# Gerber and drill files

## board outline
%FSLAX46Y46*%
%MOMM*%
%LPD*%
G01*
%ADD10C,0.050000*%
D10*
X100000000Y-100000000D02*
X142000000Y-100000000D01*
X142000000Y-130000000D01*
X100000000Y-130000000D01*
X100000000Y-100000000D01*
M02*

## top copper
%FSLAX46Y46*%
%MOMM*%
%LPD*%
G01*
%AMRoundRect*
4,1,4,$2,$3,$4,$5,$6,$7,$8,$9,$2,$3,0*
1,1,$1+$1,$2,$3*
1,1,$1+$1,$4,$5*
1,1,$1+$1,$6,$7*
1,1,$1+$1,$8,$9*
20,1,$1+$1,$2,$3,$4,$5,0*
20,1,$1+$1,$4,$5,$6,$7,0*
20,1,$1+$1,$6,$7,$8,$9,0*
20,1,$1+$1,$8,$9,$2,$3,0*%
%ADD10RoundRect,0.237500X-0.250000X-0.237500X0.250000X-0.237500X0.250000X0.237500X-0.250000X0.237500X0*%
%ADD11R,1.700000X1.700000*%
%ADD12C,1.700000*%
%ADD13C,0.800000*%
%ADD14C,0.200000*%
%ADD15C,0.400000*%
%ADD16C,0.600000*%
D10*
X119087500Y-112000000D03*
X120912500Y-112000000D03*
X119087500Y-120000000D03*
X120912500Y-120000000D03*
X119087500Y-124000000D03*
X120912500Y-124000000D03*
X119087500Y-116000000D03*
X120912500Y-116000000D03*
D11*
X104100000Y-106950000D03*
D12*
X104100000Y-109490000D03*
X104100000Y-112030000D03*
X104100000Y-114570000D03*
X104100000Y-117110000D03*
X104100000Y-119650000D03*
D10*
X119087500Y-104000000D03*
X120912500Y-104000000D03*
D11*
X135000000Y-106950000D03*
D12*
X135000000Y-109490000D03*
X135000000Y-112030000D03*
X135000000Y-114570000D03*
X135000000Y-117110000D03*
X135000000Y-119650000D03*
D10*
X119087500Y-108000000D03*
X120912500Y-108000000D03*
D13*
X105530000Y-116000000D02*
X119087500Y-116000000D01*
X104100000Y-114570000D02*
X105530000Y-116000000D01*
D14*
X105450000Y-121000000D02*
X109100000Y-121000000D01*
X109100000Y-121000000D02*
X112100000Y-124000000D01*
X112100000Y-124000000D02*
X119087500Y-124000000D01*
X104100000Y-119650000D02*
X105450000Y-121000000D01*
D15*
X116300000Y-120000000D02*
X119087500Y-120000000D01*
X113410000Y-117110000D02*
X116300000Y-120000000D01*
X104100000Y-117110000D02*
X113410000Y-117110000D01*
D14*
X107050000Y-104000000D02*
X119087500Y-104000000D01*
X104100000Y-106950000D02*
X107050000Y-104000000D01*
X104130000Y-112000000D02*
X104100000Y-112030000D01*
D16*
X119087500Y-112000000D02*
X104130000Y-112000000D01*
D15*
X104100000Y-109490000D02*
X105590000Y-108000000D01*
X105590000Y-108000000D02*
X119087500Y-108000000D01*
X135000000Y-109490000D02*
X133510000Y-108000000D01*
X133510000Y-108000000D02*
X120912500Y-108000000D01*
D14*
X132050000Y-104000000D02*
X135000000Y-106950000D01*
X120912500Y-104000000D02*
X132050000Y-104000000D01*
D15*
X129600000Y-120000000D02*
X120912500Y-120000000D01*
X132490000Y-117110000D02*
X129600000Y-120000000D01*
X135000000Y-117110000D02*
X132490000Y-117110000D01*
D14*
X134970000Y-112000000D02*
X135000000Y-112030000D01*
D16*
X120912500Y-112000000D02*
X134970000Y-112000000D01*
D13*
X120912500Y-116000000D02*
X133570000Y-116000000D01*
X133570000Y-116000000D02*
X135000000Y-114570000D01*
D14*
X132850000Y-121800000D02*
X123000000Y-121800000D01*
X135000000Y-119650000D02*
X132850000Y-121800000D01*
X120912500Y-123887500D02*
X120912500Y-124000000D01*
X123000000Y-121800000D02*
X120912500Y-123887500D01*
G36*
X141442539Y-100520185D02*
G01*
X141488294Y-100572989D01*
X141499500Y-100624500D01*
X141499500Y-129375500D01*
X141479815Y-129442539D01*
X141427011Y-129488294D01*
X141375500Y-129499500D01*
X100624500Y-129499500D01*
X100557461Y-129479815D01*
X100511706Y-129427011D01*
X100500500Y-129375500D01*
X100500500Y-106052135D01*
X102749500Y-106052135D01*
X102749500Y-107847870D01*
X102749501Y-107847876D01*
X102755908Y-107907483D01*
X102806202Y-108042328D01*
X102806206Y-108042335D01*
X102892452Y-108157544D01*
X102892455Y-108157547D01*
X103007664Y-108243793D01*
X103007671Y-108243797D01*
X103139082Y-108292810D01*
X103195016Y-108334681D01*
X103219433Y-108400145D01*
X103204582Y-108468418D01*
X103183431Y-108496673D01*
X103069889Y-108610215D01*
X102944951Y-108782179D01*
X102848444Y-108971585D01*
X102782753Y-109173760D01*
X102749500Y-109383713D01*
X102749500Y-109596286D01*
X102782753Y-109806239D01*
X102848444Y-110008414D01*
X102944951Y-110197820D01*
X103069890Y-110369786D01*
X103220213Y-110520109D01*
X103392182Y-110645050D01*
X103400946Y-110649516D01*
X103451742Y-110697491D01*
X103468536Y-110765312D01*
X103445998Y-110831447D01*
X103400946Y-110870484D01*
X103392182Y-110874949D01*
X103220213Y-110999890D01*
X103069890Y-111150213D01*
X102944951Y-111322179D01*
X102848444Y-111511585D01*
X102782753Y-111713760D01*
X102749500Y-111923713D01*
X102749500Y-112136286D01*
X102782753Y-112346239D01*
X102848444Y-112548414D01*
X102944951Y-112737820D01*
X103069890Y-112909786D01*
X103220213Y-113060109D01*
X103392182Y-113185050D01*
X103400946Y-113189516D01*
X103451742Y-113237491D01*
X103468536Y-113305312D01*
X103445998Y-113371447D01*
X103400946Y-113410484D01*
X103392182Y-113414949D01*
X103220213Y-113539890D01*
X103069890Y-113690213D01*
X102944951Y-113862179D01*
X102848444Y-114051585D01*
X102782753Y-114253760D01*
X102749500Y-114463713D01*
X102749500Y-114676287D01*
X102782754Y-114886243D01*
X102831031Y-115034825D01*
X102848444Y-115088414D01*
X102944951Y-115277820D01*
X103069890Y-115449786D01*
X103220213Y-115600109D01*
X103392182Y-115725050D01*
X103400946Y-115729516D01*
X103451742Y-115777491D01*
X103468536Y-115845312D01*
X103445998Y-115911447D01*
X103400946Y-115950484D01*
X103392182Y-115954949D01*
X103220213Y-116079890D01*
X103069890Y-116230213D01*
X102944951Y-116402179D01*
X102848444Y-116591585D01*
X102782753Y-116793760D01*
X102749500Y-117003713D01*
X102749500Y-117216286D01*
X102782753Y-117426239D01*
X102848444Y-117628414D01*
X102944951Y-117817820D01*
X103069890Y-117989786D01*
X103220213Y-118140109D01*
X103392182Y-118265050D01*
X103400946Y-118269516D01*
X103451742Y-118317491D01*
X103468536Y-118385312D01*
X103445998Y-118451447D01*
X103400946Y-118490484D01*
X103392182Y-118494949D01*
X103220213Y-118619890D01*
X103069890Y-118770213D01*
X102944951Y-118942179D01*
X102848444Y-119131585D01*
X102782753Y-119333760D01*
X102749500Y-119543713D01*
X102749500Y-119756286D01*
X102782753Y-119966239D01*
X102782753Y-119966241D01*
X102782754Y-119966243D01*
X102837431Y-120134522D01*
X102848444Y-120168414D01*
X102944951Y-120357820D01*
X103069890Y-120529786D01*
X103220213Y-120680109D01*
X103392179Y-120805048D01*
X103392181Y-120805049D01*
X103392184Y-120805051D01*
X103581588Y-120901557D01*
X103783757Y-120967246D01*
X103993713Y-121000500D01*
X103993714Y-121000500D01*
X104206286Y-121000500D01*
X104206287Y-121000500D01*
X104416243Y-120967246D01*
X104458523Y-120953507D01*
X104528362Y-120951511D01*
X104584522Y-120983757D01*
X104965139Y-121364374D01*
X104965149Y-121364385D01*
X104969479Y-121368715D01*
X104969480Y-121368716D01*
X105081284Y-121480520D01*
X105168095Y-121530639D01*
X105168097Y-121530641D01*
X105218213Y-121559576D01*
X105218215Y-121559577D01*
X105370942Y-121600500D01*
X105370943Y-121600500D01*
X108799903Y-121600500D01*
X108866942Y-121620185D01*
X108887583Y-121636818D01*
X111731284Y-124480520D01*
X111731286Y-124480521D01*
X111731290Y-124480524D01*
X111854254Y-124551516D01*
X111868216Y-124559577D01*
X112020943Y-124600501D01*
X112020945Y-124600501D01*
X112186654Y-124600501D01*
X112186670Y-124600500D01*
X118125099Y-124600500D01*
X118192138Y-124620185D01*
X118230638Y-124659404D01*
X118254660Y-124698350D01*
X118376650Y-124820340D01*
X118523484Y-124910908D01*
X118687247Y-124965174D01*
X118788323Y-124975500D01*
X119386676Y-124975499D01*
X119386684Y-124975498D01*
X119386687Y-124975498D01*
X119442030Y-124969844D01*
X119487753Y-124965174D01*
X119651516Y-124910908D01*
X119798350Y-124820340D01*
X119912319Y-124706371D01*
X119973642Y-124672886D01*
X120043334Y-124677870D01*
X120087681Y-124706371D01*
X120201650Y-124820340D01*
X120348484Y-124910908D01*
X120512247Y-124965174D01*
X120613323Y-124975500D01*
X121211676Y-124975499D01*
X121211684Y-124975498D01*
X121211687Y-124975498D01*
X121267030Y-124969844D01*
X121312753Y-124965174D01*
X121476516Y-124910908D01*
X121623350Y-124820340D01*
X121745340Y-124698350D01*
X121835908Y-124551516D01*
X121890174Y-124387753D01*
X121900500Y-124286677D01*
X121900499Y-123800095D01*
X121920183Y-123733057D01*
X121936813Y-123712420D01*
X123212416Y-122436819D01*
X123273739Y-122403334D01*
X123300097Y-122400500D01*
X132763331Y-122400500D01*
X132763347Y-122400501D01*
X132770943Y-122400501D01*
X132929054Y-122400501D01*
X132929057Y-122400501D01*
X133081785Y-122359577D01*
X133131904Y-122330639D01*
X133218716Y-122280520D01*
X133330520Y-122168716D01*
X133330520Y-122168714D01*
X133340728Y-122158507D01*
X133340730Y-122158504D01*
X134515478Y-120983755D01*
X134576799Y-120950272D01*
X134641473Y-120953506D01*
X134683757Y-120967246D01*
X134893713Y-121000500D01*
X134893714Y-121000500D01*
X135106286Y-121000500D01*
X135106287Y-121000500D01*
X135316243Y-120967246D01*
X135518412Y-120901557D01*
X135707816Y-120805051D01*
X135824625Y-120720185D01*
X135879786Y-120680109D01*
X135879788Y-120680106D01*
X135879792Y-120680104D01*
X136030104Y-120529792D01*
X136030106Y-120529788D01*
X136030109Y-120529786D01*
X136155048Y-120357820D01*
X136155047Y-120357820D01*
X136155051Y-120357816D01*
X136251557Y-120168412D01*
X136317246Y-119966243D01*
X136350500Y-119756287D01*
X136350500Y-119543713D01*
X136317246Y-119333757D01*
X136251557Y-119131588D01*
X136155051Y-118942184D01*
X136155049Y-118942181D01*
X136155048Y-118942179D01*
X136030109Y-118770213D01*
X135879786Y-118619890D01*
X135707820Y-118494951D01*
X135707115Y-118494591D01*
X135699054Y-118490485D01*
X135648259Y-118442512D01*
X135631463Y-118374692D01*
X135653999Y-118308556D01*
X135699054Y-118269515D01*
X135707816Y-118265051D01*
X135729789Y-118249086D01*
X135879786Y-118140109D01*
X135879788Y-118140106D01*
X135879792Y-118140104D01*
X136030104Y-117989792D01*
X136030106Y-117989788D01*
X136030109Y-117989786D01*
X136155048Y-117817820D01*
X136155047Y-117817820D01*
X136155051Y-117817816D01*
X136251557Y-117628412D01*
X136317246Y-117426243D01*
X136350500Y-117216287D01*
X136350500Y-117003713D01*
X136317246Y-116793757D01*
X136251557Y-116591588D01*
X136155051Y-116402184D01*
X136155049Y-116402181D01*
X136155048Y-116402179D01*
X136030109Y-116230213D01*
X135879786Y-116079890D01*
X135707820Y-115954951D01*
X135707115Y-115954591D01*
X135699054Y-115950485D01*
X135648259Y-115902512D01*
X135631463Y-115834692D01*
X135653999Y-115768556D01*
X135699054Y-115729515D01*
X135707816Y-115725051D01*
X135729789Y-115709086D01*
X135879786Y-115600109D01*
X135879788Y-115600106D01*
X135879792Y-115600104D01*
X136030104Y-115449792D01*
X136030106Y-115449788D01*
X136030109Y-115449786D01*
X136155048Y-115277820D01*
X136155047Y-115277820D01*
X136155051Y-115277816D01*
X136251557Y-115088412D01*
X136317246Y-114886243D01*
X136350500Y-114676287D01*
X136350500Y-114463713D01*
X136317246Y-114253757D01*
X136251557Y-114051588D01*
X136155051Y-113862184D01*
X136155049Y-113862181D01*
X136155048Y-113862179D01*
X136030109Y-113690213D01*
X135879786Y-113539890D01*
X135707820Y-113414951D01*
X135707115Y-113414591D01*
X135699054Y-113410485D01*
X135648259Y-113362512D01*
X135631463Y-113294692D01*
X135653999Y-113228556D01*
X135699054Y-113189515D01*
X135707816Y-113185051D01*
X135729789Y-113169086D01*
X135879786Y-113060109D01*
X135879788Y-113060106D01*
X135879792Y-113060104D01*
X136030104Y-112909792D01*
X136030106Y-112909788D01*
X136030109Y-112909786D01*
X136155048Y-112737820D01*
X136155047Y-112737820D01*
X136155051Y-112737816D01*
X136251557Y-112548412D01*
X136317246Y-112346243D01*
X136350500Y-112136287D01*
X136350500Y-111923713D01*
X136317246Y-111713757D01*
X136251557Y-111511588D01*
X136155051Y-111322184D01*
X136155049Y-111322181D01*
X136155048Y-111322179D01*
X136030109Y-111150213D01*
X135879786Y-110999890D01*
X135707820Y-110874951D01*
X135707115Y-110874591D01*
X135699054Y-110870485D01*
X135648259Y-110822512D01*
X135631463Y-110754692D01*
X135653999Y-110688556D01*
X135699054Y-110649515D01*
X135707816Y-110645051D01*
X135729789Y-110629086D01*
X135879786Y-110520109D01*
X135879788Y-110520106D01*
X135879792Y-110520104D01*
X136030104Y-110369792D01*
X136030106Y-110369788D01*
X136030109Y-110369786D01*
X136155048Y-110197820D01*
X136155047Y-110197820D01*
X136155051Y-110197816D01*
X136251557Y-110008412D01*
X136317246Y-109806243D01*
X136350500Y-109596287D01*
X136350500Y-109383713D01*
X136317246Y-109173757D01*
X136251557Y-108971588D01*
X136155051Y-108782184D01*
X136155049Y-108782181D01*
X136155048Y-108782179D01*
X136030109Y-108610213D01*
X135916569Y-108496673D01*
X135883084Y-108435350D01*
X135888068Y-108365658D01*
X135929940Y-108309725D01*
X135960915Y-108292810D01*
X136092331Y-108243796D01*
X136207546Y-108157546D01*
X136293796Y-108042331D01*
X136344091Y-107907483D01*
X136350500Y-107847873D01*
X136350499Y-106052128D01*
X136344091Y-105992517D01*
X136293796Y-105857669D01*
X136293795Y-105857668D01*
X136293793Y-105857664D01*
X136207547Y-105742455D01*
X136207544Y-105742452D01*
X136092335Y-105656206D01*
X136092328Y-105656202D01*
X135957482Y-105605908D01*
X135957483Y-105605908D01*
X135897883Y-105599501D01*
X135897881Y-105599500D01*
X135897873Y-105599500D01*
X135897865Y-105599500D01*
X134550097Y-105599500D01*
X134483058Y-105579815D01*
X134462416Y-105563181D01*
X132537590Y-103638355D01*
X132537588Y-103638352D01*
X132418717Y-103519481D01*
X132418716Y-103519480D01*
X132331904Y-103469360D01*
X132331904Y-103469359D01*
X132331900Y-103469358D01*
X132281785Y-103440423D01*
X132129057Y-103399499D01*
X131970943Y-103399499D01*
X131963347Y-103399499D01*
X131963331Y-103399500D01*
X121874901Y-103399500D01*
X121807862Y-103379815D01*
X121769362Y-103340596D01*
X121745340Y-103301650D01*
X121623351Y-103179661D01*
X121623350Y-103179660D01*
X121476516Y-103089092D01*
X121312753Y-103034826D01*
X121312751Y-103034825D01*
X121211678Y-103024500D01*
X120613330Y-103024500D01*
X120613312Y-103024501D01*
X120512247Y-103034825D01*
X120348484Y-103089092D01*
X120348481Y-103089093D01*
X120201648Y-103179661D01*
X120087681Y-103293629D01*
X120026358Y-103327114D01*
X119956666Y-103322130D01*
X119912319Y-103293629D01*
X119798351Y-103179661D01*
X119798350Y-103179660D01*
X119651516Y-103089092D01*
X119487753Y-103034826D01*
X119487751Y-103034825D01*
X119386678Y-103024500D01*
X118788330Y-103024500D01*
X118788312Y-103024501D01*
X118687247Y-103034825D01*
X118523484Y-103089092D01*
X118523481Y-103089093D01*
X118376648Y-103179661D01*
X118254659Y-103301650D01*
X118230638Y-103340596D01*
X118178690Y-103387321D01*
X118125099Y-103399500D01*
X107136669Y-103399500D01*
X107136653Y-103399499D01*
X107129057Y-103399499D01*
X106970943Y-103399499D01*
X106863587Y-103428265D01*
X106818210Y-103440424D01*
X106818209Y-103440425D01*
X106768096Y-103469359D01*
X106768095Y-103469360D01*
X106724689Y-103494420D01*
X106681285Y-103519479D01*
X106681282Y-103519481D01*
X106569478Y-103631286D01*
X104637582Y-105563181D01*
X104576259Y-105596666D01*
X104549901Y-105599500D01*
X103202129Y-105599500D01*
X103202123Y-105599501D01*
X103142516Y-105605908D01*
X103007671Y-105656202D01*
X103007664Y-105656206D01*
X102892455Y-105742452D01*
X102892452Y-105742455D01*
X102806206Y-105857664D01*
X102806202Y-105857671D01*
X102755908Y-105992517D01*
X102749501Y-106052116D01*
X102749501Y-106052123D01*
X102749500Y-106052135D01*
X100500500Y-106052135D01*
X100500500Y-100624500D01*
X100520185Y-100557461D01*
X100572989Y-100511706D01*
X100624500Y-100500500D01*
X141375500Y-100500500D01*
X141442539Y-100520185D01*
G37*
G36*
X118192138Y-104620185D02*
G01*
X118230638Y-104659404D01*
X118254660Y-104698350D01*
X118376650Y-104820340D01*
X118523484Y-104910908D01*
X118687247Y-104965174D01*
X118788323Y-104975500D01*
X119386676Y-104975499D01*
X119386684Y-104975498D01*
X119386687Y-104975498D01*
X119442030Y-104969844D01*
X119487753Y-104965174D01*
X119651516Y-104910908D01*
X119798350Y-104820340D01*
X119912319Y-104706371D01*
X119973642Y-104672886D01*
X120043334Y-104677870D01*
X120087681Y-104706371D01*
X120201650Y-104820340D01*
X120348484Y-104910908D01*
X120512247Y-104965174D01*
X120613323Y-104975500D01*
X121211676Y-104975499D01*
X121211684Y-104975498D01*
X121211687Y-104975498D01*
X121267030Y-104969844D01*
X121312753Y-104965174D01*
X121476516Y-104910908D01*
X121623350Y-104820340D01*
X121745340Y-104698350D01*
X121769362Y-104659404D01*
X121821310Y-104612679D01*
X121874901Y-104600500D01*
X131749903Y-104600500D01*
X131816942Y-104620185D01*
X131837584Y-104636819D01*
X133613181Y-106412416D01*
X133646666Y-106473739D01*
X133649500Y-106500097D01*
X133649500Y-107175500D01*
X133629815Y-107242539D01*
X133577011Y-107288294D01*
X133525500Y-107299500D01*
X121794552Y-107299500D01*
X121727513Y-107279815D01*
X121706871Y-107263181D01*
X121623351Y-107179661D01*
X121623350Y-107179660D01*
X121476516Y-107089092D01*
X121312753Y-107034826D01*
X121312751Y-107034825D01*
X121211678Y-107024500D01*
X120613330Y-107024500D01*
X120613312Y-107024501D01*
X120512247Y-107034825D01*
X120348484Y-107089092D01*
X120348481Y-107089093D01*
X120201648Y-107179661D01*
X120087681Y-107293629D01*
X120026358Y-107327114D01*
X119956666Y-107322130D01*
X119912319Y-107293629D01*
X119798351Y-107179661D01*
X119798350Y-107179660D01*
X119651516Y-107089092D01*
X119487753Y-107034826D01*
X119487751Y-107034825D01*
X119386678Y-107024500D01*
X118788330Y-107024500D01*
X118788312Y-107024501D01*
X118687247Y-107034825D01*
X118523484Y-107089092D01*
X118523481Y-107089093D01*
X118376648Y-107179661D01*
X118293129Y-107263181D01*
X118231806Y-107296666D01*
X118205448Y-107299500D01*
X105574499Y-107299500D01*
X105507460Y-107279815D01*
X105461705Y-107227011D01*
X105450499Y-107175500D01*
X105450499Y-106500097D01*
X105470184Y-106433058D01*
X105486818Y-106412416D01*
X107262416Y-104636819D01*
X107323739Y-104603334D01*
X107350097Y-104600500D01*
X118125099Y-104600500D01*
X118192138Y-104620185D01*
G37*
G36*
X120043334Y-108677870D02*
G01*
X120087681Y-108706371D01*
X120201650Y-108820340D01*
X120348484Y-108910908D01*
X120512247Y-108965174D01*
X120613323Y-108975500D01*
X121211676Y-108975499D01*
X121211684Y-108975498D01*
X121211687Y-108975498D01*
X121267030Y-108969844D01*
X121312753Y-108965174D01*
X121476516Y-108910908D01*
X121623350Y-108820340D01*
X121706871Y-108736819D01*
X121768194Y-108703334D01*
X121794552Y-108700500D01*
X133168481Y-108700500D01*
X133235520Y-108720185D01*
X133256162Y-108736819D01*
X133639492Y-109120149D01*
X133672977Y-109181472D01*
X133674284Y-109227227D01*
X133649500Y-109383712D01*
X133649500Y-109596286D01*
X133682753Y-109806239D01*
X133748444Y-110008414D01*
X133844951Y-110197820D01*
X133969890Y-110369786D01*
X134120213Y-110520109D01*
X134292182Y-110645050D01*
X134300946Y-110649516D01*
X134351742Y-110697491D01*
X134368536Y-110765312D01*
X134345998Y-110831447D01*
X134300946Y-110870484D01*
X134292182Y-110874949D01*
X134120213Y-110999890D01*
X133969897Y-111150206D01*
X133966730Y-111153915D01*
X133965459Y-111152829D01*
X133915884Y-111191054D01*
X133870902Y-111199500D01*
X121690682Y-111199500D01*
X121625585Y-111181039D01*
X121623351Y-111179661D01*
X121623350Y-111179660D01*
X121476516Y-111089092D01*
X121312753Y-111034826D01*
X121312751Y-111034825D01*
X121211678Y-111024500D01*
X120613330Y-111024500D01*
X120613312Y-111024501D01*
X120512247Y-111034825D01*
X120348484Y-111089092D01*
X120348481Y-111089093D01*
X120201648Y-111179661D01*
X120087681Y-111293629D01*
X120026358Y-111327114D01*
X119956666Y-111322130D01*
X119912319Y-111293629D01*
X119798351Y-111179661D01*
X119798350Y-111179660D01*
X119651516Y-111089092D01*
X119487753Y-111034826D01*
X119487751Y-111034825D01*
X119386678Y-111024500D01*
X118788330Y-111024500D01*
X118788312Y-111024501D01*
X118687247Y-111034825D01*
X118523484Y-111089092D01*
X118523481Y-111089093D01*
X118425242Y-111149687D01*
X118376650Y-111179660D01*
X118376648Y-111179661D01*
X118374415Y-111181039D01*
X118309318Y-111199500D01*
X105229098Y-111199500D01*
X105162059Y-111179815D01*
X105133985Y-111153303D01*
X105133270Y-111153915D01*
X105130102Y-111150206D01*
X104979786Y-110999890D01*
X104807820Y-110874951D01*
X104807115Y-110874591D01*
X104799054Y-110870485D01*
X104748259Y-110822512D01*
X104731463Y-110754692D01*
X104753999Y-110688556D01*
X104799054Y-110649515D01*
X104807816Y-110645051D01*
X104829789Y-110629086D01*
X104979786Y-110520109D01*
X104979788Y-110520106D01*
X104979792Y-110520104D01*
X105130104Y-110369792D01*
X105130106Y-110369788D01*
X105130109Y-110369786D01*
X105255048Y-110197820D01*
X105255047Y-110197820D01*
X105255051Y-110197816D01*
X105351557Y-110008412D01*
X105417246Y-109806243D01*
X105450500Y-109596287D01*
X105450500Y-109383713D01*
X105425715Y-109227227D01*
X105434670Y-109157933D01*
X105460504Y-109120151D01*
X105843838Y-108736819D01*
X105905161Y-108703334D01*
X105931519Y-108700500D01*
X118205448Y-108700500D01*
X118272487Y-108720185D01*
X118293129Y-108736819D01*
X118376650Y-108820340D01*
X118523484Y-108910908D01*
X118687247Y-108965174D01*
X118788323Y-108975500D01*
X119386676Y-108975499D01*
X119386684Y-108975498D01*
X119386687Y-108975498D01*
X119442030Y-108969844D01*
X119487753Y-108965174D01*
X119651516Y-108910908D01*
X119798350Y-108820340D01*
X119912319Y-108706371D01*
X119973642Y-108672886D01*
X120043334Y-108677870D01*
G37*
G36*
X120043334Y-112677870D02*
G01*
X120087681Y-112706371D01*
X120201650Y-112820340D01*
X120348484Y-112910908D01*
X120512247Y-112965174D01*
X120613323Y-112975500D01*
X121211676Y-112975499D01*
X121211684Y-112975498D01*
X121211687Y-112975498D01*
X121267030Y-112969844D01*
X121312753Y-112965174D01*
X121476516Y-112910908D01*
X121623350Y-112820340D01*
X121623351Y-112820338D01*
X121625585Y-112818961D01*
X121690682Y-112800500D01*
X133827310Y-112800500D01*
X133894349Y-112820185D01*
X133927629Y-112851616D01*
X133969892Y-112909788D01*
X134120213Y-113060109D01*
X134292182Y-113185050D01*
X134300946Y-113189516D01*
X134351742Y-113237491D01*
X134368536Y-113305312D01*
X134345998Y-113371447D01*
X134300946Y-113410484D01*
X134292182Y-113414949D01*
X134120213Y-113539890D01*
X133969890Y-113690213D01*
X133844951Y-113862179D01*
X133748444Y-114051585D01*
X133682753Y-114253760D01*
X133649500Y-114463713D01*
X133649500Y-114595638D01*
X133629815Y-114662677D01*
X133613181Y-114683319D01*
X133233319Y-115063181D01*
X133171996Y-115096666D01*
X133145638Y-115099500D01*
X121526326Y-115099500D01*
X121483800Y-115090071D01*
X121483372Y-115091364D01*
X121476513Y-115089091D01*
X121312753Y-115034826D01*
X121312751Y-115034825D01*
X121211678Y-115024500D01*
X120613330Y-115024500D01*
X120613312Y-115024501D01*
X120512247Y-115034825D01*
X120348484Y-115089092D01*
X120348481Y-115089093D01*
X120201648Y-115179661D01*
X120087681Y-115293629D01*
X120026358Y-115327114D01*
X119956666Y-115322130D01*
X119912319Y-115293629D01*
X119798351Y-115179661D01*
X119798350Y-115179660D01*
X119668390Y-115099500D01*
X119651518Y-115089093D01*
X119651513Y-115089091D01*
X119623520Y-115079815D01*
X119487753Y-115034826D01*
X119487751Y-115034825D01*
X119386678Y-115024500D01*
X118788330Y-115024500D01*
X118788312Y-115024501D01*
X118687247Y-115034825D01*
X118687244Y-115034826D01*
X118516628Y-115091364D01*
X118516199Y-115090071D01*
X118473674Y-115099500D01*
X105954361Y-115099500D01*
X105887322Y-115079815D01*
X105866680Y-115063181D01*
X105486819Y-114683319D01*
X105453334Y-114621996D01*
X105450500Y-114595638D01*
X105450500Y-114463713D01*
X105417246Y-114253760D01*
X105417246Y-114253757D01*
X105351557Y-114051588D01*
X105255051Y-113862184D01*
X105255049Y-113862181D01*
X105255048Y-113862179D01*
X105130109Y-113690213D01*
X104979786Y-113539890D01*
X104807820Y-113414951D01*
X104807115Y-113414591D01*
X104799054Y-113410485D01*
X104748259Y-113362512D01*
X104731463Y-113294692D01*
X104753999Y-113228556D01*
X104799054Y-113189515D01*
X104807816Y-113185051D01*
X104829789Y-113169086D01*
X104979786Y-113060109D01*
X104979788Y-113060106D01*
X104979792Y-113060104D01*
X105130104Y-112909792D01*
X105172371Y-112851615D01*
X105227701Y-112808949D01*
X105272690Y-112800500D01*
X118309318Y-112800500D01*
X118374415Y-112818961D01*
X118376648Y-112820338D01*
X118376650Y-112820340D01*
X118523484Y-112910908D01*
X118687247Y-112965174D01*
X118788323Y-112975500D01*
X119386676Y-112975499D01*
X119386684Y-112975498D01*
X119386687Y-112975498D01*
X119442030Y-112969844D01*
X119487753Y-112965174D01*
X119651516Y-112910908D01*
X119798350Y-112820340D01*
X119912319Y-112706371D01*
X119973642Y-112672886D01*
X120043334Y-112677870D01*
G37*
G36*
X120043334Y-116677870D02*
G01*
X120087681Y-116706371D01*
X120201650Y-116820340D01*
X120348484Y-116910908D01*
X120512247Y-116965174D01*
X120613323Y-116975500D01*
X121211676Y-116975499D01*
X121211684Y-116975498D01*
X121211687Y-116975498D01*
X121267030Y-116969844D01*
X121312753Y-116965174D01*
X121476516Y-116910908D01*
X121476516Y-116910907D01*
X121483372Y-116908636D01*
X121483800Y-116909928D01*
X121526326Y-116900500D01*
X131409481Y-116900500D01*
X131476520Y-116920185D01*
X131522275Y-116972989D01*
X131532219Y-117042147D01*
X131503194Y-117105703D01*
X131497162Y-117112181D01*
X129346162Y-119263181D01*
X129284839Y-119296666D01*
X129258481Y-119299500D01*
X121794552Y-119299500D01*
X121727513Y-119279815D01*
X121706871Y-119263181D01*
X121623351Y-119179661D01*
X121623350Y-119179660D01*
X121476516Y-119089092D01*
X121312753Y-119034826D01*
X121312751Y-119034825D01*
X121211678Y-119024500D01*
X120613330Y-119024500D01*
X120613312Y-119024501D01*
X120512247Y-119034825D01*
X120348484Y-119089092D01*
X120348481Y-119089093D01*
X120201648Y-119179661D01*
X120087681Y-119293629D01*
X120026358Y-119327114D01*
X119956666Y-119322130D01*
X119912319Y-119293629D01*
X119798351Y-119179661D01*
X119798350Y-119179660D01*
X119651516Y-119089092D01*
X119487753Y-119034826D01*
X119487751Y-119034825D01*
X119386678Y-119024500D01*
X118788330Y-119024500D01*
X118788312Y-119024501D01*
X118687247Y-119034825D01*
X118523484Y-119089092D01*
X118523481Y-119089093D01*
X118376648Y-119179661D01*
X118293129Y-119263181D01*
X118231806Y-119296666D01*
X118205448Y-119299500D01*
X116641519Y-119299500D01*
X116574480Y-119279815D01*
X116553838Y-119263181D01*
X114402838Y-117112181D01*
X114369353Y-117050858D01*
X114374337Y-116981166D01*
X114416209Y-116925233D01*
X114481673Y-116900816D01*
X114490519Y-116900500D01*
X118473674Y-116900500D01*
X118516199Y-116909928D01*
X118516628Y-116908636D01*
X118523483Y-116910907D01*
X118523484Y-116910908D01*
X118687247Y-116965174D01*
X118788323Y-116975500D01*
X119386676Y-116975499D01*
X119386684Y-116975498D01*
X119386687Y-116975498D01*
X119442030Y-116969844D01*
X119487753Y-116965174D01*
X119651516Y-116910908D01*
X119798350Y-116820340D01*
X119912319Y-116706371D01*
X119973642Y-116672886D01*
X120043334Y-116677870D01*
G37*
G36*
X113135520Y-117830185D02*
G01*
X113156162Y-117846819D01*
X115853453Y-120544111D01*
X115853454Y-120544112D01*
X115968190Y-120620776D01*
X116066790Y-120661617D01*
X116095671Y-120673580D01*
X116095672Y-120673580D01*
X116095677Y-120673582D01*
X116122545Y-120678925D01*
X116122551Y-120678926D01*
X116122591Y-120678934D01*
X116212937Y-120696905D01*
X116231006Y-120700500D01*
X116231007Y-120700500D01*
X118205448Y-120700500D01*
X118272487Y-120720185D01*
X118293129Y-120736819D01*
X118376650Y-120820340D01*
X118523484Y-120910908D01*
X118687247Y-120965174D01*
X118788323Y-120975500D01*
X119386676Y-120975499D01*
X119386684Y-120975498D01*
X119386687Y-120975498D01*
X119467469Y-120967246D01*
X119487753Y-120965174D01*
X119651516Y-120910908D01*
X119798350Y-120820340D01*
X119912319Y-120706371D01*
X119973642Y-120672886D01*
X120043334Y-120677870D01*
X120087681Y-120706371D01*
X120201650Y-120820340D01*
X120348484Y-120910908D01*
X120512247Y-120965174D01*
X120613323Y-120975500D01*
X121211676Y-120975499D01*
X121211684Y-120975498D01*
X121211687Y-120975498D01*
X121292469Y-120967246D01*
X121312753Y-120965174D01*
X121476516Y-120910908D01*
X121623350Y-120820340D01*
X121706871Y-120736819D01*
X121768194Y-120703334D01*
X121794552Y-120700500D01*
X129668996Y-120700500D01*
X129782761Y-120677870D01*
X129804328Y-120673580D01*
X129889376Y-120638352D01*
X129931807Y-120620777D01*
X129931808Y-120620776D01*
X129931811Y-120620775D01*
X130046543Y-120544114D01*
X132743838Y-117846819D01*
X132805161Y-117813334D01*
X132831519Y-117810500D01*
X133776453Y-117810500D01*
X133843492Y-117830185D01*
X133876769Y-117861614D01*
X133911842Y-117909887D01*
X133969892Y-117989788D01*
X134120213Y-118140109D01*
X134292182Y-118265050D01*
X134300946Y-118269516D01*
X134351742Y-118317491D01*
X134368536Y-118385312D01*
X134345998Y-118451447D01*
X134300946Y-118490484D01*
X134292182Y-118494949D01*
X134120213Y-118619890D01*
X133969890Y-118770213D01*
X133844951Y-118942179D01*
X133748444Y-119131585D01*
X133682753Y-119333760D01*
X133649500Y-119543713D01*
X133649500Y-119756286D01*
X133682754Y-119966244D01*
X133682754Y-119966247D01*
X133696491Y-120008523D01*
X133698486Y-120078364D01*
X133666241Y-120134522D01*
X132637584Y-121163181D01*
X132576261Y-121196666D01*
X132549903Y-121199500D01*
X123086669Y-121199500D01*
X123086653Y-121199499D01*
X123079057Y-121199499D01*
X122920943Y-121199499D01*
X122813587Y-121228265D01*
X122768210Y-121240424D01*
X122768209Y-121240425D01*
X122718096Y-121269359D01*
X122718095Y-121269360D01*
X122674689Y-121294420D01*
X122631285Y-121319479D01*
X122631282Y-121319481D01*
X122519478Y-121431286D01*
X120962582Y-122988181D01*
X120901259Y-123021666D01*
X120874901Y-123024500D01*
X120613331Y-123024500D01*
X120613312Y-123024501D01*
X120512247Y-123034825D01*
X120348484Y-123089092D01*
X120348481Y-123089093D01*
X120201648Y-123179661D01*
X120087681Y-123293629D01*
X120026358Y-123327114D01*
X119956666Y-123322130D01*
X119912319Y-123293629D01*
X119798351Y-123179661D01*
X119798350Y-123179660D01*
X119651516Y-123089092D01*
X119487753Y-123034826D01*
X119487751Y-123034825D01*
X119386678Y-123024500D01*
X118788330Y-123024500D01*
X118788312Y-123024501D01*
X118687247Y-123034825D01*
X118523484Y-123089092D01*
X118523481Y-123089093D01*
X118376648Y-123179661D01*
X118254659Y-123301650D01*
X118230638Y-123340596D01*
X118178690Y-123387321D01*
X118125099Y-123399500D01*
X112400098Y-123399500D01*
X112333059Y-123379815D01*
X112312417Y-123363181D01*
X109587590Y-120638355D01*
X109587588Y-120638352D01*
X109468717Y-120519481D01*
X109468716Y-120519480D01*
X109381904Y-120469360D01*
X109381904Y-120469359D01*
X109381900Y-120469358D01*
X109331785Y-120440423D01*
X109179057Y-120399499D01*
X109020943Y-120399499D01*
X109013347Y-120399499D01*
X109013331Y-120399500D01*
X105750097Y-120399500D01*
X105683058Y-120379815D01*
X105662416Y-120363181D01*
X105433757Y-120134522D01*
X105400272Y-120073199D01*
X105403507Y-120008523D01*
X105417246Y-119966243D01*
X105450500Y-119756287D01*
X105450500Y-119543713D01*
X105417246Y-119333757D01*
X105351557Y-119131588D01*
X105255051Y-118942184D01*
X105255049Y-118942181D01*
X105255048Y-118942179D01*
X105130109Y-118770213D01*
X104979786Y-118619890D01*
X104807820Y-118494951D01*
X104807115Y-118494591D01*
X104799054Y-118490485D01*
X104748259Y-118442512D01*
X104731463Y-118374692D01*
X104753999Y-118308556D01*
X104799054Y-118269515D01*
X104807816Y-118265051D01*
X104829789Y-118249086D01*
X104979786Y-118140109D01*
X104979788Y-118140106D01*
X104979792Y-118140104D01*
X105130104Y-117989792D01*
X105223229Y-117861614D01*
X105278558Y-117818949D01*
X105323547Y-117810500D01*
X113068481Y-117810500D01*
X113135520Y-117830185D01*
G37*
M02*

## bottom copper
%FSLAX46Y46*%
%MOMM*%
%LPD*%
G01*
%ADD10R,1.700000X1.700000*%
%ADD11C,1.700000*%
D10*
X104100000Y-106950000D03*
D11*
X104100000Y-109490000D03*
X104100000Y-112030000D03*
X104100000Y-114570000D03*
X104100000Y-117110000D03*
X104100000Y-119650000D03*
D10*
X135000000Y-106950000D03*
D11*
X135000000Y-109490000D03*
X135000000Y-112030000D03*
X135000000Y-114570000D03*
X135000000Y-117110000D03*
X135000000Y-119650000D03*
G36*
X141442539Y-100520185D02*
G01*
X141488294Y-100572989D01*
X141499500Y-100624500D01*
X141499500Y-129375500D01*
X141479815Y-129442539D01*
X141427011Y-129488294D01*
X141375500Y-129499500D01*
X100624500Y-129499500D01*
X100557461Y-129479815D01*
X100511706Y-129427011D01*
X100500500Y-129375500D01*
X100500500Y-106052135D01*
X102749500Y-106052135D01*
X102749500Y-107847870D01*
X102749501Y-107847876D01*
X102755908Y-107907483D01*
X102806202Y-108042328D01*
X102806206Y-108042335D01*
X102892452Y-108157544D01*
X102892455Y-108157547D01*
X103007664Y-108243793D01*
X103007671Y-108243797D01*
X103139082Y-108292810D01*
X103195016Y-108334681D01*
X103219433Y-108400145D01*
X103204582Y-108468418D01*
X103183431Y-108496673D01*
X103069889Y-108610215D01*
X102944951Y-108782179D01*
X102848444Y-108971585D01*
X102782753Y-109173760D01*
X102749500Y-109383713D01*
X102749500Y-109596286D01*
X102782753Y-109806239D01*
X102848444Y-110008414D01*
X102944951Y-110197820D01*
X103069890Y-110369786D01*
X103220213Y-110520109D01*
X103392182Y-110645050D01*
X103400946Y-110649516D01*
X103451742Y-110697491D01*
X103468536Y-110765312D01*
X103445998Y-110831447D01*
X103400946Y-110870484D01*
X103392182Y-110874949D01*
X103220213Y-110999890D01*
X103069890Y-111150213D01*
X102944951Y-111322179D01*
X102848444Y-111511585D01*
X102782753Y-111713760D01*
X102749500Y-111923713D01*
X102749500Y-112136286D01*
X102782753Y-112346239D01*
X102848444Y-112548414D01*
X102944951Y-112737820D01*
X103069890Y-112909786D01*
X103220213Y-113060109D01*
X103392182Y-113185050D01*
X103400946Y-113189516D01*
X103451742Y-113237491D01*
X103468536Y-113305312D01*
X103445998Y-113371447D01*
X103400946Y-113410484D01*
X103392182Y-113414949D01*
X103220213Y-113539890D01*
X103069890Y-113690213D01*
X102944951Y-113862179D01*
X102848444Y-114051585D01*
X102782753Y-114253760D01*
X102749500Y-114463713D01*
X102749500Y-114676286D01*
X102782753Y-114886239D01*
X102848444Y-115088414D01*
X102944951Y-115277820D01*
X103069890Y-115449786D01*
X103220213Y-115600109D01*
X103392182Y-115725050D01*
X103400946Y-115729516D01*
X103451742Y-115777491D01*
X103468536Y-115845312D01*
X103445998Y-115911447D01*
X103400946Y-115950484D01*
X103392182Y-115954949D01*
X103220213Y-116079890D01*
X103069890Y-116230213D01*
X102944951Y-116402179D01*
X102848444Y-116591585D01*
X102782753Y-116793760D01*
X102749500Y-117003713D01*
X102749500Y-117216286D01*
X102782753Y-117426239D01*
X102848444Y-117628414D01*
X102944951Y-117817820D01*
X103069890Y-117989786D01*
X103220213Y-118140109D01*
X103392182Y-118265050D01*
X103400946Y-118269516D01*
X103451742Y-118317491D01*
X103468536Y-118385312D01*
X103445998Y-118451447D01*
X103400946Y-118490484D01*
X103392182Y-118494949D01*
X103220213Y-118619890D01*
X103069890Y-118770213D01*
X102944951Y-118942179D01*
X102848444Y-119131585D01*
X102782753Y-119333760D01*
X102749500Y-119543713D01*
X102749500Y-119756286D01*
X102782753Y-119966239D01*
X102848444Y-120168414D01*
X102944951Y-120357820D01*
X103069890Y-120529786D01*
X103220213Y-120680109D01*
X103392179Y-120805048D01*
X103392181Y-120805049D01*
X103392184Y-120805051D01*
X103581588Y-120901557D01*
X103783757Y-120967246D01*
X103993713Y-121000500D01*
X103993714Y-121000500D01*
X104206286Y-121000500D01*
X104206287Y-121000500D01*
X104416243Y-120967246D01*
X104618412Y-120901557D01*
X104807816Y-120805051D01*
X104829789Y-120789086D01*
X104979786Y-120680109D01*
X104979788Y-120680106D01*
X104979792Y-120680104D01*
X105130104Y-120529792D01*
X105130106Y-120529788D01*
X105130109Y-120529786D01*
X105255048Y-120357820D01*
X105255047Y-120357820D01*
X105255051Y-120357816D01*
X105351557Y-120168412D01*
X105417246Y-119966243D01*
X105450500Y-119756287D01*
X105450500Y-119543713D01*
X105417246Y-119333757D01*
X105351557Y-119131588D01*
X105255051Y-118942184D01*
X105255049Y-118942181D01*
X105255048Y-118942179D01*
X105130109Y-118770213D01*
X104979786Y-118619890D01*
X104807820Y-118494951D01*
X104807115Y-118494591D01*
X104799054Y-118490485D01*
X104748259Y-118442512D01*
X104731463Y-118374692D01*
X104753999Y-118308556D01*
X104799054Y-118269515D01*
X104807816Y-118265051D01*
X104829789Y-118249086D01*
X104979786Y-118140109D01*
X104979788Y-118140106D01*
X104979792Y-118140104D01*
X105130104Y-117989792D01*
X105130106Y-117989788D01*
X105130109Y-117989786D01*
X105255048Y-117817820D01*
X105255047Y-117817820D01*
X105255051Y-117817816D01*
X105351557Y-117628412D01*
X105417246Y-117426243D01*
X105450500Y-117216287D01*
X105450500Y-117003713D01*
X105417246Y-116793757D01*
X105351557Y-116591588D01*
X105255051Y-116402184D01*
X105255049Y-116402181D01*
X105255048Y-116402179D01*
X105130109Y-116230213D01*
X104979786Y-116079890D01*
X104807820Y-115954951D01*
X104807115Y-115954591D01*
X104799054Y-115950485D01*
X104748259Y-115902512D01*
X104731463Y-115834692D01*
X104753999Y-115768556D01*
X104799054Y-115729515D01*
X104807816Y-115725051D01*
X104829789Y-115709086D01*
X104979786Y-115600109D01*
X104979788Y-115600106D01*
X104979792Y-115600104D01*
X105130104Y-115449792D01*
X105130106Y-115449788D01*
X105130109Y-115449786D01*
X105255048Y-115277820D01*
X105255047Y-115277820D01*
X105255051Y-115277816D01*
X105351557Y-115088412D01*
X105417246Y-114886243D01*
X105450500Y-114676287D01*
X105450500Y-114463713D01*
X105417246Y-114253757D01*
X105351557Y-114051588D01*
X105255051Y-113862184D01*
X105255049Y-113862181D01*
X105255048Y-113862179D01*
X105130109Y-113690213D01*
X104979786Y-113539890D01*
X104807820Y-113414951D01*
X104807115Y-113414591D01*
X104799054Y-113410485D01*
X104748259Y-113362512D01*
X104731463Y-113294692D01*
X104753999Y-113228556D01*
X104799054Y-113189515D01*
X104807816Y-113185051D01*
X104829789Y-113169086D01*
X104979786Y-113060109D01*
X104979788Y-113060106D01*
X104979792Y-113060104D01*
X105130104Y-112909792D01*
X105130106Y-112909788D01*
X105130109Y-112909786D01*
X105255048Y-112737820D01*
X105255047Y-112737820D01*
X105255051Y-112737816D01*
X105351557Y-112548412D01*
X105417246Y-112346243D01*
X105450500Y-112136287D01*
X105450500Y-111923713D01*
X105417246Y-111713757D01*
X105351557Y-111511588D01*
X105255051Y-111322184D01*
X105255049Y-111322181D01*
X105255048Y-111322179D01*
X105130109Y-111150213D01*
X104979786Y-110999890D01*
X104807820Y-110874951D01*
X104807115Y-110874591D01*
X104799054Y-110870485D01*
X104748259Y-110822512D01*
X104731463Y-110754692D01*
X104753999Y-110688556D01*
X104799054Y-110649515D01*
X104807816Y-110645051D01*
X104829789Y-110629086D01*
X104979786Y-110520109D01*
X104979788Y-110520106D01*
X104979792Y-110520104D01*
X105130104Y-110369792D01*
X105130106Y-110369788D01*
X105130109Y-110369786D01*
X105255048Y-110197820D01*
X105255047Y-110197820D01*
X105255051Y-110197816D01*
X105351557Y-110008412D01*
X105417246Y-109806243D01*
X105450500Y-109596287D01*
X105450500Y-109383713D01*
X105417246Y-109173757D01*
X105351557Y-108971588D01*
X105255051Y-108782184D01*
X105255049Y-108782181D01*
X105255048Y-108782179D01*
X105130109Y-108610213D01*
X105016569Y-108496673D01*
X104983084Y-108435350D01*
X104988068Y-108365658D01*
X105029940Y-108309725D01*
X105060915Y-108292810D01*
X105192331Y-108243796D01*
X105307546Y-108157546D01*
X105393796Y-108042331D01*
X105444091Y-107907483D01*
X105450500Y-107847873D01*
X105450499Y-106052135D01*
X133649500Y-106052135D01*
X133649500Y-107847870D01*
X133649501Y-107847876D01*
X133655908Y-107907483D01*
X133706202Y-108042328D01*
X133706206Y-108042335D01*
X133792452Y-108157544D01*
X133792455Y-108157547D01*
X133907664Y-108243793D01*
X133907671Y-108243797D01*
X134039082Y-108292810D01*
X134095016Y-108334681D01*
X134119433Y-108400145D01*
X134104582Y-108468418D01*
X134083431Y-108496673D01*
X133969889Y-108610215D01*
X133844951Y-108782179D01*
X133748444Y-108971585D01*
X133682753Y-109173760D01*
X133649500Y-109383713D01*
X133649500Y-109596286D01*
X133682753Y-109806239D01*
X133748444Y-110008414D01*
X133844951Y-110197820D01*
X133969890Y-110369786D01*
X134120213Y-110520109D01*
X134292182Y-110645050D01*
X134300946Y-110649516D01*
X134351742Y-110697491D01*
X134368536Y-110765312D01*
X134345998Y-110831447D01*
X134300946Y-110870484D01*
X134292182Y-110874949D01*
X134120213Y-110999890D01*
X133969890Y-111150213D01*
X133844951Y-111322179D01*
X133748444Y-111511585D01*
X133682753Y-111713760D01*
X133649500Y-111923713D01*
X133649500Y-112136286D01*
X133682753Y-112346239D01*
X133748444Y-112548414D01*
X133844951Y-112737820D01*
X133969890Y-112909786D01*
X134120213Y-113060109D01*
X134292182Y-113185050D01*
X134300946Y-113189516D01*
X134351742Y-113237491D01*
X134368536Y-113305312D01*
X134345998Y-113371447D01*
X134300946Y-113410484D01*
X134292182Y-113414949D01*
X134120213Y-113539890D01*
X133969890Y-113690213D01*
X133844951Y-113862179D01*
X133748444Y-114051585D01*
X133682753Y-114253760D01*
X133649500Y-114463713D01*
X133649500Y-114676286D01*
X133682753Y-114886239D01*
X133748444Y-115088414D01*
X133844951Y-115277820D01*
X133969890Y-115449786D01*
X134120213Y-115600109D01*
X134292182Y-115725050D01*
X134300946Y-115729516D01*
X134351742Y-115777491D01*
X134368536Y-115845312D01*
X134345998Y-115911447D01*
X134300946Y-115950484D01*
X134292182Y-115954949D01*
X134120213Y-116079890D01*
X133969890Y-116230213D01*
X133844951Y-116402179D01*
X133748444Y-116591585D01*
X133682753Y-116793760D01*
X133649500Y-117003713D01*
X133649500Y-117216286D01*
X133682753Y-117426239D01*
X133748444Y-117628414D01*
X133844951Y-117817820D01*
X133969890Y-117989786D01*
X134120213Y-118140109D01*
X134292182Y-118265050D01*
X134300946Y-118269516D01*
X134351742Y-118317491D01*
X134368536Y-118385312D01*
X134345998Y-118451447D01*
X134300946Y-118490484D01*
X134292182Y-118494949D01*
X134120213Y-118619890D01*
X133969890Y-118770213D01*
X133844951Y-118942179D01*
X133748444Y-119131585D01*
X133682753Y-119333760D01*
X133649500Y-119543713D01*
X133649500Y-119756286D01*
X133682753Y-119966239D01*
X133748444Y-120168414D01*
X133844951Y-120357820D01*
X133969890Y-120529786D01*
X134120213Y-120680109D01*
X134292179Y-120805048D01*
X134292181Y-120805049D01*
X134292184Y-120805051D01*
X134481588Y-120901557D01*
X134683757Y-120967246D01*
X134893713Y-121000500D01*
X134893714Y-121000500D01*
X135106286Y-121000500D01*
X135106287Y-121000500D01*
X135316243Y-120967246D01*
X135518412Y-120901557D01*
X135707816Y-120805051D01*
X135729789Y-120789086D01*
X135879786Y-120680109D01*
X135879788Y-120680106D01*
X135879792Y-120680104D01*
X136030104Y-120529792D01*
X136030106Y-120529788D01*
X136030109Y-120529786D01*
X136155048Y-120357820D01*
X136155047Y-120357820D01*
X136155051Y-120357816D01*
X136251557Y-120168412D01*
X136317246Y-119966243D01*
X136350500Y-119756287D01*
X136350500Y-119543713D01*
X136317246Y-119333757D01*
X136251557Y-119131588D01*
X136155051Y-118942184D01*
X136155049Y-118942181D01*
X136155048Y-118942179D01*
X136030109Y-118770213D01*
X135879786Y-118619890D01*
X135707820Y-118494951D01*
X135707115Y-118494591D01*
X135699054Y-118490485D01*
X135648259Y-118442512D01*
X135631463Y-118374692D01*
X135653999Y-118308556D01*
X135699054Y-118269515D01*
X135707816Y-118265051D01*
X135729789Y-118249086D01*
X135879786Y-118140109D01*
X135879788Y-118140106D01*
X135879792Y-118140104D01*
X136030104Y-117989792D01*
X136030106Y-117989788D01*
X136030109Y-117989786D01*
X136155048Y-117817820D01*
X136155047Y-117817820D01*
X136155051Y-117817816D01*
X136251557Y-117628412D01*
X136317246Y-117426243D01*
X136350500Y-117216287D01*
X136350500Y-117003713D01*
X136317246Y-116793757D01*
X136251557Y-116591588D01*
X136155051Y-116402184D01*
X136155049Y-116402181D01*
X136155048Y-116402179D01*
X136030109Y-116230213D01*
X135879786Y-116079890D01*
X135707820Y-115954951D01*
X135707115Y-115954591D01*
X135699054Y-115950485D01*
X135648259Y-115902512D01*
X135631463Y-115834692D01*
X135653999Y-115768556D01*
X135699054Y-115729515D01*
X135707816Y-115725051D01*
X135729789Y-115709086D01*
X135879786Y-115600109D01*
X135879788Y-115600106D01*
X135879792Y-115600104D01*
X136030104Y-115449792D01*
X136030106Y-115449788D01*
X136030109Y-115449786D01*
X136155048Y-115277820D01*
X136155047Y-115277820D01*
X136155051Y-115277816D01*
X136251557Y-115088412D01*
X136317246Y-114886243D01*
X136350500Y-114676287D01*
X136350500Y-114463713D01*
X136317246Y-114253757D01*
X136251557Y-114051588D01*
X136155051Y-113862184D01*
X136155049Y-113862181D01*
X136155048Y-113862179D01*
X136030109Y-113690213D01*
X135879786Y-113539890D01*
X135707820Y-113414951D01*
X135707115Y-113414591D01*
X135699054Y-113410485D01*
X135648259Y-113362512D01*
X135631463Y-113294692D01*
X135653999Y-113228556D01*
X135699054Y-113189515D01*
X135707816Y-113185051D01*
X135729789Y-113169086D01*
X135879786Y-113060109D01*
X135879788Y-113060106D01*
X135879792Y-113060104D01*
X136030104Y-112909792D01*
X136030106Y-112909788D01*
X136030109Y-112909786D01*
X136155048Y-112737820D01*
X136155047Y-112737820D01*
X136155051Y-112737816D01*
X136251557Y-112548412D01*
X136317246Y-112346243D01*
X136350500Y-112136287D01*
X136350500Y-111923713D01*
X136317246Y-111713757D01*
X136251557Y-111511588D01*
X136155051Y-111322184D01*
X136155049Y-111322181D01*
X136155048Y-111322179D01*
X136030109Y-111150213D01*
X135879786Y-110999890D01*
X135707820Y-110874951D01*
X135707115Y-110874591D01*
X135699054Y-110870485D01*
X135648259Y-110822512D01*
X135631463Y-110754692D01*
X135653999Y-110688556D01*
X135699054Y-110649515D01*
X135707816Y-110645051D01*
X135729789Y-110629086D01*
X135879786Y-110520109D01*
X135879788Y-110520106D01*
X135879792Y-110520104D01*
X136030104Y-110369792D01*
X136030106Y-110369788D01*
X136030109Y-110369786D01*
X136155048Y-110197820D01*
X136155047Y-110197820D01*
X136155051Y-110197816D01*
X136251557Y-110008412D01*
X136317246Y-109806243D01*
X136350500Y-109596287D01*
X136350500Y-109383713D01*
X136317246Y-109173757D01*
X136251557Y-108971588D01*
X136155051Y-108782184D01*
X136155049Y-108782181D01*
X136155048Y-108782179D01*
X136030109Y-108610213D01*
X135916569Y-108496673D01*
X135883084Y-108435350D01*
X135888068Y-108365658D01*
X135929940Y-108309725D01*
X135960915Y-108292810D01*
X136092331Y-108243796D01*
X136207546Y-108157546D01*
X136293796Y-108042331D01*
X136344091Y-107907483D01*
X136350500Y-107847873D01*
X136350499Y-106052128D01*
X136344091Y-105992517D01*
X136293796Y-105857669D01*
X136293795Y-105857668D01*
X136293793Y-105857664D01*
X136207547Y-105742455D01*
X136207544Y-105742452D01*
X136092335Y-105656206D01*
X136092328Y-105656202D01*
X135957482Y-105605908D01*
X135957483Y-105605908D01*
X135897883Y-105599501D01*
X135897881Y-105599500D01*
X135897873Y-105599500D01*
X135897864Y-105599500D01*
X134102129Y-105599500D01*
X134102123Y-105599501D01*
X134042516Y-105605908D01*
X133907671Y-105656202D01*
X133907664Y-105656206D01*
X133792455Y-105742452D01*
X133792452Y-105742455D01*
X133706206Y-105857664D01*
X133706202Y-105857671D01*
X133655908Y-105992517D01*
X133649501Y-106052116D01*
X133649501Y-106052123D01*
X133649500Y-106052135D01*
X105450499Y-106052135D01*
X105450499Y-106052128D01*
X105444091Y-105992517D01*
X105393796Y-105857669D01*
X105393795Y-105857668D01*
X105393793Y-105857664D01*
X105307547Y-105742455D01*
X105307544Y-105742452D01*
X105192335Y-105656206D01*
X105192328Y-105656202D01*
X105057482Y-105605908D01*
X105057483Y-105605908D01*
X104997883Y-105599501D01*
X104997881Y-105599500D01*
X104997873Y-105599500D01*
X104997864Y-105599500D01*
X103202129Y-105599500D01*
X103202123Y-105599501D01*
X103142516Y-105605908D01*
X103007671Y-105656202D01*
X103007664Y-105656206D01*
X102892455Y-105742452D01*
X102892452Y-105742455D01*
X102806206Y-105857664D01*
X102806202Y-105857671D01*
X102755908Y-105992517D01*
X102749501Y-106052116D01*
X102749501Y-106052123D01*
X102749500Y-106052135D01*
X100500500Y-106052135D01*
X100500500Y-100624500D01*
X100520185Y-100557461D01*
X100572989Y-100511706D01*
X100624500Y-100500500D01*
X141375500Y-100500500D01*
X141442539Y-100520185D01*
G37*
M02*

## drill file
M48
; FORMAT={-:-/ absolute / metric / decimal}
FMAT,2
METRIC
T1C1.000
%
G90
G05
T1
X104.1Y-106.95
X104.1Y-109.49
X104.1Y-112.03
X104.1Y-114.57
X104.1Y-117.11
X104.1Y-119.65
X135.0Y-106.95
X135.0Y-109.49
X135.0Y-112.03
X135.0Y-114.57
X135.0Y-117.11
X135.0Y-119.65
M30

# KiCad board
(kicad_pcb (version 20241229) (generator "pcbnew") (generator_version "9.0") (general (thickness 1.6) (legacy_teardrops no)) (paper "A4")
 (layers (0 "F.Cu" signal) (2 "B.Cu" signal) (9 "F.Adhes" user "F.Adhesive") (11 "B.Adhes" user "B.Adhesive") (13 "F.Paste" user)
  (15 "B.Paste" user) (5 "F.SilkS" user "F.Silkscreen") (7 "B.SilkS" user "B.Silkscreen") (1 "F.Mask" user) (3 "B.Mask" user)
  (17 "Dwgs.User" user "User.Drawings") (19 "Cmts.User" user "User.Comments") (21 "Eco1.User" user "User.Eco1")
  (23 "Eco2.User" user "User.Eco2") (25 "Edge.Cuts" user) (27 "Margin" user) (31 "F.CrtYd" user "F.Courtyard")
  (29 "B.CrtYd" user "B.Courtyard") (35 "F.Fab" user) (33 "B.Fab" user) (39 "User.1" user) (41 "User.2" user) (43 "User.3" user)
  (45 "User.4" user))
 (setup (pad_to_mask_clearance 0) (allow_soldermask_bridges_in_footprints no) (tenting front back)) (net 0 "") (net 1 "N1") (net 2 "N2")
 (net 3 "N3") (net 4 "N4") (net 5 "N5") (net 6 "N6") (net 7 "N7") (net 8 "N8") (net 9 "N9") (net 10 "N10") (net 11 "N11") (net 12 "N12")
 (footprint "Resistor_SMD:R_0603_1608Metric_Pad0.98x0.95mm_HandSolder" (layer "F.Cu") (at 120 112)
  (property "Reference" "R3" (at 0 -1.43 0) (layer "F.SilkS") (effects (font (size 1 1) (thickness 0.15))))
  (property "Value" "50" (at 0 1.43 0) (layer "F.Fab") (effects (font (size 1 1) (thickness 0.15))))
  (pad "1" smd roundrect (at -0.9125 0) (size 0.975 0.95) (layers "F.Cu" "F.Mask" "F.Paste") (roundrect_rratio 0.25) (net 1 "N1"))
  (pad "2" smd roundrect (at 0.9125 0) (size 0.975 0.95) (layers "F.Cu" "F.Mask" "F.Paste") (roundrect_rratio 0.25) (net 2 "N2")))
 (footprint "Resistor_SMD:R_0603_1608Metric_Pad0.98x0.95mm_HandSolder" (layer "F.Cu") (at 120 120)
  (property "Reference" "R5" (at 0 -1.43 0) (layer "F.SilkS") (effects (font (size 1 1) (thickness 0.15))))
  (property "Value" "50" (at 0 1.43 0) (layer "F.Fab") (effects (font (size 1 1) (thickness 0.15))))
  (pad "1" smd roundrect (at -0.9125 0) (size 0.975 0.95) (layers "F.Cu" "F.Mask" "F.Paste") (roundrect_rratio 0.25) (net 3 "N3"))
  (pad "2" smd roundrect (at 0.9125 0) (size 0.975 0.95) (layers "F.Cu" "F.Mask" "F.Paste") (roundrect_rratio 0.25) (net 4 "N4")))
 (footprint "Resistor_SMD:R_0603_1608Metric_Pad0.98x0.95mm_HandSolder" (layer "F.Cu") (at 120 124)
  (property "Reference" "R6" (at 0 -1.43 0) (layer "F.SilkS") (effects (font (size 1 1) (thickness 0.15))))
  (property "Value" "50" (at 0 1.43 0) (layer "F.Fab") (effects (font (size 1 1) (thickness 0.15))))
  (pad "1" smd roundrect (at -0.9125 0) (size 0.975 0.95) (layers "F.Cu" "F.Mask" "F.Paste") (roundrect_rratio 0.25) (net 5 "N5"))
  (pad "2" smd roundrect (at 0.9125 0) (size 0.975 0.95) (layers "F.Cu" "F.Mask" "F.Paste") (roundrect_rratio 0.25) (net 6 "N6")))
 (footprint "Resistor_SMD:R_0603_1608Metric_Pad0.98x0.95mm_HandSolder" (layer "F.Cu") (at 120 116)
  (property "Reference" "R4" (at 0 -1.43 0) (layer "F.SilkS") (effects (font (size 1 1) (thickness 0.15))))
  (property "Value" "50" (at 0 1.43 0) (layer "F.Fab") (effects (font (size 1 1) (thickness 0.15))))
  (pad "1" smd roundrect (at -0.9125 0) (size 0.975 0.95) (layers "F.Cu" "F.Mask" "F.Paste") (roundrect_rratio 0.25) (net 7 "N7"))
  (pad "2" smd roundrect (at 0.9125 0) (size 0.975 0.95) (layers "F.Cu" "F.Mask" "F.Paste") (roundrect_rratio 0.25) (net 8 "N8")))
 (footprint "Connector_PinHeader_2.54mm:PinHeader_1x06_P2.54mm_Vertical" (layer "F.Cu") (at 104.1 106.95)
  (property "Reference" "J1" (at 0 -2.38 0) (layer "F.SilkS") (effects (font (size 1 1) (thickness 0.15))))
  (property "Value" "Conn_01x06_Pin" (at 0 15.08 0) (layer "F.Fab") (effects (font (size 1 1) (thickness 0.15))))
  (pad "1" thru_hole rect (at 0 0) (size 1.7 1.7) (drill 1) (layers "*.Cu" "*.Mask") (remove_unused_layers no) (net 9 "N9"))
  (pad "2" thru_hole circle (at 0 2.54) (size 1.7 1.7) (drill 1) (layers "*.Cu" "*.Mask") (remove_unused_layers no) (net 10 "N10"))
  (pad "3" thru_hole circle (at 0 5.08) (size 1.7 1.7) (drill 1) (layers "*.Cu" "*.Mask") (remove_unused_layers no) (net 1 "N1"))
  (pad "4" thru_hole circle (at 0 7.62) (size 1.7 1.7) (drill 1) (layers "*.Cu" "*.Mask") (remove_unused_layers no) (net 7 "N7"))
  (pad "5" thru_hole circle (at 0 10.16) (size 1.7 1.7) (drill 1) (layers "*.Cu" "*.Mask") (remove_unused_layers no) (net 3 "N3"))
  (pad "6" thru_hole circle (at 0 12.7) (size 1.7 1.7) (drill 1) (layers "*.Cu" "*.Mask") (remove_unused_layers no) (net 5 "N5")))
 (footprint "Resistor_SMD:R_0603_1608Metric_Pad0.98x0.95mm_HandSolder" (layer "F.Cu") (at 120 104)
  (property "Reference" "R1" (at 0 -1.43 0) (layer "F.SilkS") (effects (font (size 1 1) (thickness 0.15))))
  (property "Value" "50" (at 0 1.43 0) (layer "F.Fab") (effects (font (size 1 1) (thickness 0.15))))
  (pad "1" smd roundrect (at -0.9125 0) (size 0.975 0.95) (layers "F.Cu" "F.Mask" "F.Paste") (roundrect_rratio 0.25) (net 9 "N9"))
  (pad "2" smd roundrect (at 0.9125 0) (size 0.975 0.95) (layers "F.Cu" "F.Mask" "F.Paste") (roundrect_rratio 0.25) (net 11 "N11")))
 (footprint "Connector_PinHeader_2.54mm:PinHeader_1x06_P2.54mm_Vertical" (layer "F.Cu") (at 135 106.95)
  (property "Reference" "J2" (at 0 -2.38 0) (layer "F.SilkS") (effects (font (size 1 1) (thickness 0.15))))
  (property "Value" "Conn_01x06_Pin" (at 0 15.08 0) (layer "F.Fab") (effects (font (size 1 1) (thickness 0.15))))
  (pad "1" thru_hole rect (at 0 0) (size 1.7 1.7) (drill 1) (layers "*.Cu" "*.Mask") (remove_unused_layers no) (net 11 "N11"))
  (pad "2" thru_hole circle (at 0 2.54) (size 1.7 1.7) (drill 1) (layers "*.Cu" "*.Mask") (remove_unused_layers no) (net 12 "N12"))
  (pad "3" thru_hole circle (at 0 5.08) (size 1.7 1.7) (drill 1) (layers "*.Cu" "*.Mask") (remove_unused_layers no) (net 2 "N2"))
  (pad "4" thru_hole circle (at 0 7.62) (size 1.7 1.7) (drill 1) (layers "*.Cu" "*.Mask") (remove_unused_layers no) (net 8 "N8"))
  (pad "5" thru_hole circle (at 0 10.16) (size 1.7 1.7) (drill 1) (layers "*.Cu" "*.Mask") (remove_unused_layers no) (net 4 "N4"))
  (pad "6" thru_hole circle (at 0 12.7) (size 1.7 1.7) (drill 1) (layers "*.Cu" "*.Mask") (remove_unused_layers no) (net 6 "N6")))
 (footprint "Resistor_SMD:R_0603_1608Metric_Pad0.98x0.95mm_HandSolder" (layer "F.Cu") (at 120 108)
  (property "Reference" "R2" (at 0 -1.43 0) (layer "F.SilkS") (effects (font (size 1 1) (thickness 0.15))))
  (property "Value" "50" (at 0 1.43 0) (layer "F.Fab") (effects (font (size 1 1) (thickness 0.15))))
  (pad "1" smd roundrect (at -0.9125 0) (size 0.975 0.95) (layers "F.Cu" "F.Mask" "F.Paste") (roundrect_rratio 0.25) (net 10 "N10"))
  (pad "2" smd roundrect (at 0.9125 0) (size 0.975 0.95) (layers "F.Cu" "F.Mask" "F.Paste") (roundrect_rratio 0.25) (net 12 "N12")))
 (gr_rect (start 100 100) (end 142 130) (stroke (width 0.05) (type default)) (fill no) (layer "Edge.Cuts"))
 (segment (start 105.53 116) (end 119.0875 116) (width 0.8) (layer "F.Cu") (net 7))
 (segment (start 104.1 114.57) (end 105.53 116) (width 0.8) (layer "F.Cu") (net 7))
 (segment (start 105.45 121) (end 109.1 121) (width 0.2) (layer "F.Cu") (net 5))
 (segment (start 109.1 121) (end 112.1 124) (width 0.2) (layer "F.Cu") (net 5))
 (segment (start 112.1 124) (end 119.0875 124) (width 0.2) (layer "F.Cu") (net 5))
 (segment (start 104.1 119.65) (end 105.45 121) (width 0.2) (layer "F.Cu") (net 5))
 (segment (start 116.3 120) (end 119.0875 120) (width 0.4) (layer "F.Cu") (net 3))
 (segment (start 113.41 117.11) (end 116.3 120) (width 0.4) (layer "F.Cu") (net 3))
 (segment (start 104.1 117.11) (end 113.41 117.11) (width 0.4) (layer "F.Cu") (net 3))
 (segment (start 107.05 104) (end 119.0875 104) (width 0.2) (layer "F.Cu") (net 9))
 (segment (start 104.1 106.95) (end 107.05 104) (width 0.2) (layer "F.Cu") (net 9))
 (segment (start 104.13 112) (end 104.1 112.03) (width 0.2) (layer "F.Cu") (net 1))
 (segment (start 119.0875 112) (end 104.13 112) (width 0.6) (layer "F.Cu") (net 1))
 (segment (start 104.1 109.49) (end 105.59 108) (width 0.4) (layer "F.Cu") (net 10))
 (segment (start 105.59 108) (end 119.0875 108) (width 0.4) (layer "F.Cu") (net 10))
 (segment (start 135 109.49) (end 133.51 108) (width 0.4) (layer "F.Cu") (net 12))
 (segment (start 133.51 108) (end 120.9125 108) (width 0.4) (layer "F.Cu") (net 12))
 (segment (start 132.05 104) (end 135 106.95) (width 0.2) (layer "F.Cu") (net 11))
 (segment (start 120.9125 104) (end 132.05 104) (width 0.2) (layer "F.Cu") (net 11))
 (segment (start 129.6 120) (end 120.9125 120) (width 0.4) (layer "F.Cu") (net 4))
 (segment (start 132.49 117.11) (end 129.6 120) (width 0.4) (layer "F.Cu") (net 4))
 (segment (start 135 117.11) (end 132.49 117.11) (width 0.4) (layer "F.Cu") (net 4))
 (segment (start 134.97 112) (end 135 112.03) (width 0.2) (layer "F.Cu") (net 2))
 (segment (start 120.9125 112) (end 134.97 112) (width 0.6) (layer "F.Cu") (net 2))
 (segment (start 120.9125 116) (end 133.57 116) (width 0.8) (layer "F.Cu") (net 8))
 (segment (start 133.57 116) (end 135 114.57) (width 0.8) (layer "F.Cu") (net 8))
 (segment (start 132.85 121.8) (end 123 121.8) (width 0.2) (layer "F.Cu") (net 6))
 (segment (start 135 119.65) (end 132.85 121.8) (width 0.2) (layer "F.Cu") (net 6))
 (segment (start 120.9125 123.8875) (end 120.9125 124) (width 0.2) (layer "F.Cu") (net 6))
 (segment (start 123 121.8) (end 120.9125 123.8875) (width 0.2) (layer "F.Cu") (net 6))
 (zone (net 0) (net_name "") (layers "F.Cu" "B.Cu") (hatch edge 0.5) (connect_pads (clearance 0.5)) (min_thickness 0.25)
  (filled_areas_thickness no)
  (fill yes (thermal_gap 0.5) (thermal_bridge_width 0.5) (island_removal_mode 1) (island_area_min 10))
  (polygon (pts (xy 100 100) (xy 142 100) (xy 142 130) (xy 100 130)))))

